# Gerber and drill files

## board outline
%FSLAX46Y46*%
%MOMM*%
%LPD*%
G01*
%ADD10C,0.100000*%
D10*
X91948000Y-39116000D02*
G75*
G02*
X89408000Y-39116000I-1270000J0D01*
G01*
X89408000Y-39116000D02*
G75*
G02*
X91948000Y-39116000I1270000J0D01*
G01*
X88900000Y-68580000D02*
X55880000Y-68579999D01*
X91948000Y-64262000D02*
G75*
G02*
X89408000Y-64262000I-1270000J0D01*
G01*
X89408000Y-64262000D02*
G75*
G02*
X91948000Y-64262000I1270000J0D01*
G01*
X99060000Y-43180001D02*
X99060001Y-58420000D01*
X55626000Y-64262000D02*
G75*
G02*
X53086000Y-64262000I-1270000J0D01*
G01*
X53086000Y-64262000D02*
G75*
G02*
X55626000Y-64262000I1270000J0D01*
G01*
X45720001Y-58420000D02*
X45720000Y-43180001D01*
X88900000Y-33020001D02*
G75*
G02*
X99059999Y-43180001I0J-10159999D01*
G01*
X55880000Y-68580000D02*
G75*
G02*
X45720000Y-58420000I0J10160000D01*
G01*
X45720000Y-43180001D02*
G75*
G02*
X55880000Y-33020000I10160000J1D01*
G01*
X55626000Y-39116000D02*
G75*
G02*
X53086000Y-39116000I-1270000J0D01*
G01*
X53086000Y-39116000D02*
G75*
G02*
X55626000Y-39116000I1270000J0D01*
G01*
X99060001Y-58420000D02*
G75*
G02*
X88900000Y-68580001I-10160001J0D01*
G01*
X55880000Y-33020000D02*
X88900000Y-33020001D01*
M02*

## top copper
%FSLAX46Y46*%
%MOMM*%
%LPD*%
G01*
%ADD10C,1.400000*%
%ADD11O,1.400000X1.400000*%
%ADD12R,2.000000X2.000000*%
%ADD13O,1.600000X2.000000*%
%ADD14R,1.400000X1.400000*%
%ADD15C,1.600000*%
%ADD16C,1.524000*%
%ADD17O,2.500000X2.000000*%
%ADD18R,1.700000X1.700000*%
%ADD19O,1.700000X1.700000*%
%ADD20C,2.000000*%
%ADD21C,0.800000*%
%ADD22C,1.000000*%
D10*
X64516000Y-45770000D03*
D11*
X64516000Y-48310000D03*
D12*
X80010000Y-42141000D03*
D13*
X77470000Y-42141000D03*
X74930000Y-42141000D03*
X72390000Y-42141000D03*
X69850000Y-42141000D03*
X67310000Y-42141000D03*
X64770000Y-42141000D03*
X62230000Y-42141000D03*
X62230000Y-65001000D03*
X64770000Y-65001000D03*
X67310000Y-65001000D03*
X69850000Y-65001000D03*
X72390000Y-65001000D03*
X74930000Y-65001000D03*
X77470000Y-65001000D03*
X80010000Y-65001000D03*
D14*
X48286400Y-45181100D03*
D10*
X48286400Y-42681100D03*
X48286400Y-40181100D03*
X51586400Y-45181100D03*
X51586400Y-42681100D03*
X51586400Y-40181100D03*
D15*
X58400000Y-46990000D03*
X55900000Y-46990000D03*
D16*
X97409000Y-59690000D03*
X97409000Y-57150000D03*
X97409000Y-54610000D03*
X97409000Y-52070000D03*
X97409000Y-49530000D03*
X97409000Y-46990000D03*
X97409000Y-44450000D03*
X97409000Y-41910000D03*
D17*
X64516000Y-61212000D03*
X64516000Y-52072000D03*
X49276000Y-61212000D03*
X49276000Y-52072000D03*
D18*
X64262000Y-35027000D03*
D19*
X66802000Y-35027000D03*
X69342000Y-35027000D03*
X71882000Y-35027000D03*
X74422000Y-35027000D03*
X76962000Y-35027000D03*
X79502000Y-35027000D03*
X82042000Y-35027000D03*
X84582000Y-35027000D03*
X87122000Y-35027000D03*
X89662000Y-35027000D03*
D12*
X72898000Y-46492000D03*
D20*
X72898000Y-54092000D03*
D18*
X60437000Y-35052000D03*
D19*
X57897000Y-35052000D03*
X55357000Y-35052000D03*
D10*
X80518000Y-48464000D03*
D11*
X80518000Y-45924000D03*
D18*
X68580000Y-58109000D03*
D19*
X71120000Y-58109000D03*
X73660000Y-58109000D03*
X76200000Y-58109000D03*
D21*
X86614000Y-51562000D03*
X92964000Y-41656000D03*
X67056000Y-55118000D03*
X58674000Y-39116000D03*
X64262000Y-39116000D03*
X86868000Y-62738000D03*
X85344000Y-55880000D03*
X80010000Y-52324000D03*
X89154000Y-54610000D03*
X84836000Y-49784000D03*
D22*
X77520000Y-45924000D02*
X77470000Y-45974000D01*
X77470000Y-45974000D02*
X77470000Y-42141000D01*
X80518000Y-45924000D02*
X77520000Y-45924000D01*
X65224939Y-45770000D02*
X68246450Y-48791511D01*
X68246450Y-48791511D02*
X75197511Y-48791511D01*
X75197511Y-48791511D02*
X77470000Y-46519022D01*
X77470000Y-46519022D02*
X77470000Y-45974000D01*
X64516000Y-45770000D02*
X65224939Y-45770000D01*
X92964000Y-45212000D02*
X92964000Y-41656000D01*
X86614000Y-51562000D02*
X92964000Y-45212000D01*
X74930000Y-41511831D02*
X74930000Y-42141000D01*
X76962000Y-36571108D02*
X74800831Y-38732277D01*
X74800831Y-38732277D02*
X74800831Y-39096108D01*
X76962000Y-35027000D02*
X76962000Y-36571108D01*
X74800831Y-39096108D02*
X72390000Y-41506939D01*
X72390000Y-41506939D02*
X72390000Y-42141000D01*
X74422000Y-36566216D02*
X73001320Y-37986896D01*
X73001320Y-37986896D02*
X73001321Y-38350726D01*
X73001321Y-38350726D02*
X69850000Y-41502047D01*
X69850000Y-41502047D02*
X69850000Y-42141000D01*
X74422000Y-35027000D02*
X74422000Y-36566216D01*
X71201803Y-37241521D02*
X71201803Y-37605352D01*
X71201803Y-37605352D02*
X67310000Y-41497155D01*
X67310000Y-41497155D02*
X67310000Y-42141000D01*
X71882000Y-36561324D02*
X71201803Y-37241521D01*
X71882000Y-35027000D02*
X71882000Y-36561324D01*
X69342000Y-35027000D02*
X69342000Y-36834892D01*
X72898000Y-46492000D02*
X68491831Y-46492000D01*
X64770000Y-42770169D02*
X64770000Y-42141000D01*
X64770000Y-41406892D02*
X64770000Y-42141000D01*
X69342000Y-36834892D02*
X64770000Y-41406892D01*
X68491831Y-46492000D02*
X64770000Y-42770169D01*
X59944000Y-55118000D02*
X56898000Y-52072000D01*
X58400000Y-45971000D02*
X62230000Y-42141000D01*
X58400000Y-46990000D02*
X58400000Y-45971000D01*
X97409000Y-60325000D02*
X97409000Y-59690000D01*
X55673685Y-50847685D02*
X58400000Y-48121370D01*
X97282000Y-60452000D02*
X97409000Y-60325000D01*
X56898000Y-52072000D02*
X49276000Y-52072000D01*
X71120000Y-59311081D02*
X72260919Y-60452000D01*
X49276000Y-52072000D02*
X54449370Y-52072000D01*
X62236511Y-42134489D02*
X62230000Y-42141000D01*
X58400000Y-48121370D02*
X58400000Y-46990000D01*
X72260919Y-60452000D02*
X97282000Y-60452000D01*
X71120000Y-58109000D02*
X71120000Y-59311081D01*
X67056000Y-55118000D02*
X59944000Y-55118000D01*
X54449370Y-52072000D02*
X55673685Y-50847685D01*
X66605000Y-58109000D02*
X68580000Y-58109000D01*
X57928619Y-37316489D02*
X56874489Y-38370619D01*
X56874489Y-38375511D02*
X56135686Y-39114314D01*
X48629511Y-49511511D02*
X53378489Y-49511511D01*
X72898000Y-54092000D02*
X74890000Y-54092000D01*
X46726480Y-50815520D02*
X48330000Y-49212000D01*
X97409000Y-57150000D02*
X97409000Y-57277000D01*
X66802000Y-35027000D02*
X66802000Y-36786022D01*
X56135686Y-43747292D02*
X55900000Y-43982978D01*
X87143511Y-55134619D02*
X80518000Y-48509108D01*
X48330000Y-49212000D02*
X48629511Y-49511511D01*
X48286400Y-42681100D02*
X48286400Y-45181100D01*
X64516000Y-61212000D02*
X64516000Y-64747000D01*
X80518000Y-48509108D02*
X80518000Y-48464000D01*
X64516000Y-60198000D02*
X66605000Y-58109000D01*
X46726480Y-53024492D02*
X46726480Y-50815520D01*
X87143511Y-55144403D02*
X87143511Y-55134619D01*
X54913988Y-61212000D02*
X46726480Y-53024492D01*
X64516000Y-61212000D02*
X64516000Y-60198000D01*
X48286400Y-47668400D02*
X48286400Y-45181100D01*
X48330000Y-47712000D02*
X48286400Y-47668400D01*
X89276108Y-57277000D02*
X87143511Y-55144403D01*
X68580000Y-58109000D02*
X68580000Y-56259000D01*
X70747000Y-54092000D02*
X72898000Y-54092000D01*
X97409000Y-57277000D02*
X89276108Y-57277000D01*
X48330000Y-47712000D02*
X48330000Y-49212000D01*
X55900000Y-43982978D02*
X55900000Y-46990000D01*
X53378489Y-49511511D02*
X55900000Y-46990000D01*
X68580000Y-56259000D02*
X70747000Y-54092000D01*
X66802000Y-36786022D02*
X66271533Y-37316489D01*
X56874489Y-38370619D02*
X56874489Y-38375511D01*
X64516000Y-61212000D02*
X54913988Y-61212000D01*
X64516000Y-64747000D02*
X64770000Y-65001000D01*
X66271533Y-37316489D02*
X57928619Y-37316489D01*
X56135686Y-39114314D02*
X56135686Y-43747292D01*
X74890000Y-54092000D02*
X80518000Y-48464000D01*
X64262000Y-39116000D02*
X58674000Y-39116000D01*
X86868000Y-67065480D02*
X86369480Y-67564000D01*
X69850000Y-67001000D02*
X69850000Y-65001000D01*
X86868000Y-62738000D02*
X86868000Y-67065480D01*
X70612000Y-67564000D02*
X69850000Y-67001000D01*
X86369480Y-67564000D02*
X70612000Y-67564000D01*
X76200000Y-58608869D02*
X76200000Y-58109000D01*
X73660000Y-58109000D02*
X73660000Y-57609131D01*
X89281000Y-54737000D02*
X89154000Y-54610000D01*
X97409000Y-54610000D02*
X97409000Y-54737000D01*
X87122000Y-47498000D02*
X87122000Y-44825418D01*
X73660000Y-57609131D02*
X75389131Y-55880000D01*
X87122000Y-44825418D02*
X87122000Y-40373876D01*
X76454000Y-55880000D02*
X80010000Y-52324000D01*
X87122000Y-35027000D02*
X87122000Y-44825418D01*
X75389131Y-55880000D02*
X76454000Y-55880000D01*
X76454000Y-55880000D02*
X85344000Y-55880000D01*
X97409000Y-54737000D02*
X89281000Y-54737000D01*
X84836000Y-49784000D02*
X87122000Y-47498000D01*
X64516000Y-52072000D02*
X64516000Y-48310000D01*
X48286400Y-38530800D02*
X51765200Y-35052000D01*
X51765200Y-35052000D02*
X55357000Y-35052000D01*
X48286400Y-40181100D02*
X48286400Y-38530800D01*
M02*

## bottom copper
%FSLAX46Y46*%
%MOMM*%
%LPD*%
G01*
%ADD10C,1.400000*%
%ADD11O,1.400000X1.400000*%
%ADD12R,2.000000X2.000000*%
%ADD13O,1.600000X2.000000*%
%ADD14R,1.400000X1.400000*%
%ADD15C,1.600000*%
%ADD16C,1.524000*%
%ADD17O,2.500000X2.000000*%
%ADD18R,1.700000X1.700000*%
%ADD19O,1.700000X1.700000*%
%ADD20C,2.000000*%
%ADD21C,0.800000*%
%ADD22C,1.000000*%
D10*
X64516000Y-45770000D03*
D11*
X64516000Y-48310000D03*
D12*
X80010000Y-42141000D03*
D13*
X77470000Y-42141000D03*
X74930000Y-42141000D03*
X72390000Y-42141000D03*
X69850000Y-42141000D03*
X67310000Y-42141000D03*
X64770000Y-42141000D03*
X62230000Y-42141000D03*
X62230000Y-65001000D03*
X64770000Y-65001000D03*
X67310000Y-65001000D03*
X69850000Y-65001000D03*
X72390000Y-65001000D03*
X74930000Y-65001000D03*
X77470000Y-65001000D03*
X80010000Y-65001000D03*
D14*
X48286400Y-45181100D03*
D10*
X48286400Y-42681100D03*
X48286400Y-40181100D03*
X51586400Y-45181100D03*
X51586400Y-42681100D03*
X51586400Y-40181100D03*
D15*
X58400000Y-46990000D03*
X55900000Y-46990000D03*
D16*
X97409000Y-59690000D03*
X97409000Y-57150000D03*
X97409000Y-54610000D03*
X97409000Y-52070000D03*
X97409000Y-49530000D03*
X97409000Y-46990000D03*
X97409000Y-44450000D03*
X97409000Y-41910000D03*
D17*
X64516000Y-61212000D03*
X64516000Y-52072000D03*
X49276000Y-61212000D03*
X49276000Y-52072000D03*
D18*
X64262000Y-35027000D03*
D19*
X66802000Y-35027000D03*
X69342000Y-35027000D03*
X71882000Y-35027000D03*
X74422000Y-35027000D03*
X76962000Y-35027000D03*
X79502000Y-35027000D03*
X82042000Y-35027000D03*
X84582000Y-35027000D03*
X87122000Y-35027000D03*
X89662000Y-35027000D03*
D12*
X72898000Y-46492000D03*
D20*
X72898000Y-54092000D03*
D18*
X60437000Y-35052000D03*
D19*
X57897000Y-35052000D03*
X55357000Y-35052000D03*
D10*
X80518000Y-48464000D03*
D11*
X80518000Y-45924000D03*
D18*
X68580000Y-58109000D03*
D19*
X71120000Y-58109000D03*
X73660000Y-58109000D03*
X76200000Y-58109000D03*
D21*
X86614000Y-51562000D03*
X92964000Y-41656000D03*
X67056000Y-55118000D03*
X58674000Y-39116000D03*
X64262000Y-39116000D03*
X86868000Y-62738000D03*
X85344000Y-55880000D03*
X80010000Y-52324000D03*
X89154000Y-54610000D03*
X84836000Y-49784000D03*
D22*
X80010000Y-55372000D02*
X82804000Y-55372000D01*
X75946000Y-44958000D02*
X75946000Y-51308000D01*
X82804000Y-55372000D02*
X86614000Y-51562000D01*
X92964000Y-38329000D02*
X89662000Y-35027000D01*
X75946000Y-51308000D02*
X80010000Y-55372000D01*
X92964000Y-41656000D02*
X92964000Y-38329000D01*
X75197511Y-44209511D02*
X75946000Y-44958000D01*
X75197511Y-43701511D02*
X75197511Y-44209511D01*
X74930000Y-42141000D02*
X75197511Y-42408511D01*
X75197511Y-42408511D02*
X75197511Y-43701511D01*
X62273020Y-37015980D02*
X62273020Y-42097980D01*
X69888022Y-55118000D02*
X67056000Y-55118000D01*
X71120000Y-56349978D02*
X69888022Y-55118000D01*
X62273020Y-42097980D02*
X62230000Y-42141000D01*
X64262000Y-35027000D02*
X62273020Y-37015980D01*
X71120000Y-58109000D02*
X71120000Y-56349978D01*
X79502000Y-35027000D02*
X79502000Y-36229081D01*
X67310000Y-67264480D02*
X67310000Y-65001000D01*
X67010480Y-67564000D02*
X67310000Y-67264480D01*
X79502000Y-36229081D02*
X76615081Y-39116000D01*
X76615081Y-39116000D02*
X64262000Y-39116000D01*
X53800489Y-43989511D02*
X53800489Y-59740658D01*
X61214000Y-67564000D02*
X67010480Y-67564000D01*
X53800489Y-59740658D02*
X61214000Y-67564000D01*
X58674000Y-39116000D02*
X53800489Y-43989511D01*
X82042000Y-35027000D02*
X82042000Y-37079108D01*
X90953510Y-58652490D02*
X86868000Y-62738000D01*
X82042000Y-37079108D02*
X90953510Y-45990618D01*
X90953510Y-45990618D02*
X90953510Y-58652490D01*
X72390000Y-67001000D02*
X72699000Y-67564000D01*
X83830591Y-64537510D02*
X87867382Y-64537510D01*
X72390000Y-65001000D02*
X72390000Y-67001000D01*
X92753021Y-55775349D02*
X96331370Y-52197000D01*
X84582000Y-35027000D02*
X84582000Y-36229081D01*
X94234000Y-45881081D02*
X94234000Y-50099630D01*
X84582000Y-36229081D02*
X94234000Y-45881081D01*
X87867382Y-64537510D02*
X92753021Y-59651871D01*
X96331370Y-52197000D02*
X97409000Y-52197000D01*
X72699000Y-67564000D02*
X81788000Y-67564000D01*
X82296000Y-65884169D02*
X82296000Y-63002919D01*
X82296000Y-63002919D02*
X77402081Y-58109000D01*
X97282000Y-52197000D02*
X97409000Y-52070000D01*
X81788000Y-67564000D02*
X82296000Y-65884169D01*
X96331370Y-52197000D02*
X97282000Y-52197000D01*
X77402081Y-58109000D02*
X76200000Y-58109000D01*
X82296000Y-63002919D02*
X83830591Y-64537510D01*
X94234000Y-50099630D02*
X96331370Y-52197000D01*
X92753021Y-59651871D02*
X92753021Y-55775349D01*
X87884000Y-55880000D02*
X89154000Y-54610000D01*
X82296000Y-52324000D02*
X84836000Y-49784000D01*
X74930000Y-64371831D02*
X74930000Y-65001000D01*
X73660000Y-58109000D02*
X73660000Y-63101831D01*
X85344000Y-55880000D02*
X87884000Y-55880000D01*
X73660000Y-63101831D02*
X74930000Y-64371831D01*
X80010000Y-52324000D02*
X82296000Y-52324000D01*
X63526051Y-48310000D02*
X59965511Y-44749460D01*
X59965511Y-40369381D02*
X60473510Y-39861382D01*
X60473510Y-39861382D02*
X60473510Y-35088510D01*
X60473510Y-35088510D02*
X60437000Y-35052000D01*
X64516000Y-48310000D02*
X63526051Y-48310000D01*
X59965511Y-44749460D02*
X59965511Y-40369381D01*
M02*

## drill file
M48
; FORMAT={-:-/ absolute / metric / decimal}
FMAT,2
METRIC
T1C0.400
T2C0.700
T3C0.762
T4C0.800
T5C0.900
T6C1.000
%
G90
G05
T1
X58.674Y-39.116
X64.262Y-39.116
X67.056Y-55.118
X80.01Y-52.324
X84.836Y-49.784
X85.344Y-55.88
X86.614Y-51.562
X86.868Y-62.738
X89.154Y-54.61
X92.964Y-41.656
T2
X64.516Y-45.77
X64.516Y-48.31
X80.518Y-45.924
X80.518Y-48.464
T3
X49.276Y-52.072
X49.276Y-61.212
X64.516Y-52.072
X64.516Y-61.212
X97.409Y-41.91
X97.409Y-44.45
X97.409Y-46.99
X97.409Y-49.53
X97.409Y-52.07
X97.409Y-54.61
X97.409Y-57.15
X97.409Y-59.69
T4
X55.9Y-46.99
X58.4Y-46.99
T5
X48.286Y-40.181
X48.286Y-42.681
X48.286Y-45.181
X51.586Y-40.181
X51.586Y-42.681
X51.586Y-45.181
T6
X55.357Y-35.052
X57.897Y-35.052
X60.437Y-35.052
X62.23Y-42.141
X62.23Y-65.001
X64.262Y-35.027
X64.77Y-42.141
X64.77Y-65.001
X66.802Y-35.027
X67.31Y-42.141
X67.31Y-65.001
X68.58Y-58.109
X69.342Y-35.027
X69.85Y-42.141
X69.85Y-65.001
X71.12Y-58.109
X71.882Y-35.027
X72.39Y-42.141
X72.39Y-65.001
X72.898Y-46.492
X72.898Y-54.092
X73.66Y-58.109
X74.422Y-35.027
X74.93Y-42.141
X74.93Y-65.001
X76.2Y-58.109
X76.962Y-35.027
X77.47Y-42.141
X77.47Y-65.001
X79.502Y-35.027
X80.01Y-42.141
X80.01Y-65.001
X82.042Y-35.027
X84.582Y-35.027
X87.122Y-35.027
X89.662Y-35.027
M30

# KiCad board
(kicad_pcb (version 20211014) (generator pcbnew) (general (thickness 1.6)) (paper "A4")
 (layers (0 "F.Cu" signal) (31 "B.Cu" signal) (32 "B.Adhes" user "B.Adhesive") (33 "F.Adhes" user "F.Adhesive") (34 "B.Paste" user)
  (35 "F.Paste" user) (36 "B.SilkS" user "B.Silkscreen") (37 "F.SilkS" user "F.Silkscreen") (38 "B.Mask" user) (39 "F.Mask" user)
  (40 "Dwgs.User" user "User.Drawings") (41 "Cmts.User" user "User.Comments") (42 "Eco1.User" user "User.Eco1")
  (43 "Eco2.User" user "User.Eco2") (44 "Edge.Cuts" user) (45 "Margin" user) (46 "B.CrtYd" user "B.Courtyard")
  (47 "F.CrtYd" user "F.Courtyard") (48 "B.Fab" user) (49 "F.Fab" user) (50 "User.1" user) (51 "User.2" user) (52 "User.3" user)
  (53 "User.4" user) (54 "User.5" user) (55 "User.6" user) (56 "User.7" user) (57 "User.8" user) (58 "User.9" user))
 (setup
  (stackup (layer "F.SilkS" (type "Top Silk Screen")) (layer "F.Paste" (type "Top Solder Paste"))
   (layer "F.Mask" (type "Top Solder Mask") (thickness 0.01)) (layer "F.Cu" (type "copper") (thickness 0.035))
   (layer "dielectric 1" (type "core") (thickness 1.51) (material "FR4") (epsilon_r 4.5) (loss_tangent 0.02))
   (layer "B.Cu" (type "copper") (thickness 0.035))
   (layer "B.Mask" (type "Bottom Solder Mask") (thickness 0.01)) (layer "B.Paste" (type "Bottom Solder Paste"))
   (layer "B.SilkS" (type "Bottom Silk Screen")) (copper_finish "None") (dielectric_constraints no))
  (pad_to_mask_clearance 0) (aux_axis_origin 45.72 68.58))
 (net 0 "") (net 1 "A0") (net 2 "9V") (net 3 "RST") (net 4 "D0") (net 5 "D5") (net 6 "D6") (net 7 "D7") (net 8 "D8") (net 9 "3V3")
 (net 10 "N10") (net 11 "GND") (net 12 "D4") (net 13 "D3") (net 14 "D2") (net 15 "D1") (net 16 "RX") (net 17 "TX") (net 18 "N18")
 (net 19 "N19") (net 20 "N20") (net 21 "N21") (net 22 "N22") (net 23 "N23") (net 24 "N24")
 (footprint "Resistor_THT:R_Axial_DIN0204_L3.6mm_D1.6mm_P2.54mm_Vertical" (layer "F.Cu") (at 64.516 45.77 -90)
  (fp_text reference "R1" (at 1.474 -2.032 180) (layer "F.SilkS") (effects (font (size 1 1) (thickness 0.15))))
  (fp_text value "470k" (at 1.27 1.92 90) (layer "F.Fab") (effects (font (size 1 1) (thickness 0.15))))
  (pad "1" thru_hole circle (at 0 0 270) (size 1.4 1.4) (drill 0.7) (layers *.Cu *.Mask) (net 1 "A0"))
  (pad "2" thru_hole oval (at 2.54 0 270) (size 1.4 1.4) (drill 0.7) (layers *.Cu *.Mask) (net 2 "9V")))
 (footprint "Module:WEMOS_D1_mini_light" (layer "F.Cu") (at 80.01 42.141 -90)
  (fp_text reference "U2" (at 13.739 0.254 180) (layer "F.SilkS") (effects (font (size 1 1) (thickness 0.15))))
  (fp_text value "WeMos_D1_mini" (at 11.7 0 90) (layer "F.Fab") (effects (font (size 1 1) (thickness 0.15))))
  (pad "1" thru_hole rect (at 0 0 270) (size 2 2) (drill 1) (layers *.Cu *.Mask) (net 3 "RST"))
  (pad "2" thru_hole oval (at 0 2.54 270) (size 2 1.6) (drill 1) (layers *.Cu *.Mask) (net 1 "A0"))
  (pad "3" thru_hole oval (at 0 5.08 270) (size 2 1.6) (drill 1) (layers *.Cu *.Mask) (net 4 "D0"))
  (pad "4" thru_hole oval (at 0 7.62 270) (size 2 1.6) (drill 1) (layers *.Cu *.Mask) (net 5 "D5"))
  (pad "5" thru_hole oval (at 0 10.16 270) (size 2 1.6) (drill 1) (layers *.Cu *.Mask) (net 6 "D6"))
  (pad "6" thru_hole oval (at 0 12.7 270) (size 2 1.6) (drill 1) (layers *.Cu *.Mask) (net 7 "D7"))
  (pad "7" thru_hole oval (at 0 15.24 270) (size 2 1.6) (drill 1) (layers *.Cu *.Mask) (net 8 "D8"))
  (pad "8" thru_hole oval (at 0 17.78 270) (size 2 1.6) (drill 1) (layers *.Cu *.Mask) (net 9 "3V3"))
  (pad "9" thru_hole oval (at 22.86 17.78 270) (size 2 1.6) (drill 1) (layers *.Cu *.Mask) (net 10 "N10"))
  (pad "10" thru_hole oval (at 22.86 15.24 270) (size 2 1.6) (drill 1) (layers *.Cu *.Mask) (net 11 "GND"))
  (pad "11" thru_hole oval (at 22.86 12.7 270) (size 2 1.6) (drill 1) (layers *.Cu *.Mask) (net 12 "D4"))
  (pad "12" thru_hole oval (at 22.86 10.16 270) (size 2 1.6) (drill 1) (layers *.Cu *.Mask) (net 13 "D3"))
  (pad "13" thru_hole oval (at 22.86 7.62 270) (size 2 1.6) (drill 1) (layers *.Cu *.Mask) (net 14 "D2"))
  (pad "14" thru_hole oval (at 22.86 5.08 270) (size 2 1.6) (drill 1) (layers *.Cu *.Mask) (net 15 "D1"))
  (pad "15" thru_hole oval (at 22.86 2.54 270) (size 2 1.6) (drill 1) (layers *.Cu *.Mask) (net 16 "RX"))
  (pad "16" thru_hole oval (at 22.86 0 270) (size 2 1.6) (drill 1) (layers *.Cu *.Mask) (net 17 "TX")))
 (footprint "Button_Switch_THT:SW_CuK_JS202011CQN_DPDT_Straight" (layer "F.Cu") (at 48.2864 45.1811 90)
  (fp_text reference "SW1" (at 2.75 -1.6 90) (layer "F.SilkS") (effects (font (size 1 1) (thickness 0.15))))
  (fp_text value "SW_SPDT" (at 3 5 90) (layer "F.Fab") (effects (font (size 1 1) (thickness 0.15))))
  (pad "1" thru_hole rect (at 0 0 90) (size 1.4 1.4) (drill 0.9) (layers *.Cu *.Mask) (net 11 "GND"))
  (pad "2" thru_hole circle (at 2.5 0 90) (size 1.4 1.4) (drill 0.9) (layers *.Cu *.Mask) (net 11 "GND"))
  (pad "3" thru_hole circle (at 5 0 90) (size 1.4 1.4) (drill 0.9) (layers *.Cu *.Mask) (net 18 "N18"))
  (pad "4" thru_hole circle (at 0 3.3 90) (size 1.4 1.4) (drill 0.9) (layers *.Cu *.Mask))
  (pad "5" thru_hole circle (at 2.5 3.3 90) (size 1.4 1.4) (drill 0.9) (layers *.Cu *.Mask))
  (pad "6" thru_hole circle (at 5 3.3 90) (size 1.4 1.4) (drill 0.9) (layers *.Cu *.Mask)))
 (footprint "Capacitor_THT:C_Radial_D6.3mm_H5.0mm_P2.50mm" (layer "F.Cu") (at 58.4 46.99 180)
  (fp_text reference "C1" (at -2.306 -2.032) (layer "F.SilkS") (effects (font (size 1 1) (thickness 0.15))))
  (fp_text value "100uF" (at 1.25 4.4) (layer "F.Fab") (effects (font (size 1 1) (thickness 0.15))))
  (pad "1" thru_hole circle (at 0 0 180) (size 1.6 1.6) (drill 0.8) (layers *.Cu *.Mask) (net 9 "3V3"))
  (pad "2" thru_hole circle (at 2.5 0 180) (size 1.6 1.6) (drill 0.8) (layers *.Cu *.Mask) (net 11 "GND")))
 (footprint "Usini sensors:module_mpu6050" (layer "F.Cu") (at 97.409 41.91 180)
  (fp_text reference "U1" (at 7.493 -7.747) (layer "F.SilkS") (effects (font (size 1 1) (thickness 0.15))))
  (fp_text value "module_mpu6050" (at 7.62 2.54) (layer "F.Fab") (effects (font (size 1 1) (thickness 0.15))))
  (pad "1" thru_hole circle locked (at 0 -17.78 180) (size 1.524 1.524) (drill 0.762) (layers *.Cu *.Mask) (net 9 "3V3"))
  (pad "2" thru_hole circle locked (at 0 -15.24 180) (size 1.524 1.524) (drill 0.762) (layers *.Cu *.Mask) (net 11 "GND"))
  (pad "3" thru_hole circle locked (at 0 -12.7 180) (size 1.524 1.524) (drill 0.762) (layers *.Cu *.Mask) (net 15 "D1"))
  (pad "4" thru_hole circle locked (at 0 -10.16 180) (size 1.524 1.524) (drill 0.762) (layers *.Cu *.Mask) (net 14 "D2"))
  (pad "5" thru_hole circle locked (at 0 -7.62 180) (size 1.524 1.524) (drill 0.762) (layers *.Cu *.Mask) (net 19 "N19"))
  (pad "6" thru_hole circle locked (at 0 -5.08 180) (size 1.524 1.524) (drill 0.762) (layers *.Cu *.Mask) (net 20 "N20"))
  (pad "7" thru_hole circle locked (at 0 -2.54 180) (size 1.524 1.524) (drill 0.762) (layers *.Cu *.Mask) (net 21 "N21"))
  (pad "8" thru_hole circle locked (at 0 0 180) (size 1.524 1.524) (drill 0.762) (layers *.Cu *.Mask) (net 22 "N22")))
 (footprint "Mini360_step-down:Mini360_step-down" (layer "F.Cu") (at 56.896 56.642 180)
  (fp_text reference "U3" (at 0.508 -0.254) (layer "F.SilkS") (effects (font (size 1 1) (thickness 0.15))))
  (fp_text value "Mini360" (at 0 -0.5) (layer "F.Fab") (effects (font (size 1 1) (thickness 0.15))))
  (pad "1" thru_hole oval locked (at -7.62 -4.57 180) (size 2.5 2) (drill 0.762) (layers *.Cu *.Mask) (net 11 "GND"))
  (pad "2" thru_hole oval locked (at -7.62 4.57 180) (size 2.5 2) (drill 0.762) (layers *.Cu *.Mask) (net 2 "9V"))
  (pad "3" thru_hole oval locked (at 7.62 -4.57 180) (size 2.5 2) (drill 0.762) (layers *.Cu *.Mask) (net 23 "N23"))
  (pad "4" thru_hole oval locked (at 7.62 4.57 180) (size 2.5 2) (drill 0.762) (layers *.Cu *.Mask) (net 9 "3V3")))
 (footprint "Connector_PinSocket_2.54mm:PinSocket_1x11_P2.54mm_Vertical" (layer "F.Cu") (at 64.262 35.027 90)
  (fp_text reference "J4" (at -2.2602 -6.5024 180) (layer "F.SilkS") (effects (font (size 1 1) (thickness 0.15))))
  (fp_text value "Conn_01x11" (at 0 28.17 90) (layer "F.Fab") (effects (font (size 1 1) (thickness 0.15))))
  (pad "1" thru_hole rect (at 0 0 90) (size 1.7 1.7) (drill 1) (layers *.Cu *.Mask) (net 9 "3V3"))
  (pad "2" thru_hole oval (at 0 2.54 90) (size 1.7 1.7) (drill 1) (layers *.Cu *.Mask) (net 11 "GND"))
  (pad "3" thru_hole oval (at 0 5.08 90) (size 1.7 1.7) (drill 1) (layers *.Cu *.Mask) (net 8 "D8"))
  (pad "4" thru_hole oval (at 0 7.62 90) (size 1.7 1.7) (drill 1) (layers *.Cu *.Mask) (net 7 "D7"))
  (pad "5" thru_hole oval (at 0 10.16 90) (size 1.7 1.7) (drill 1) (layers *.Cu *.Mask) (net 6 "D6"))
  (pad "6" thru_hole oval (at 0 12.7 90) (size 1.7 1.7) (drill 1) (layers *.Cu *.Mask) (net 5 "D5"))
  (pad "7" thru_hole oval (at 0 15.24 90) (size 1.7 1.7) (drill 1) (layers *.Cu *.Mask) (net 12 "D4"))
  (pad "8" thru_hole oval (at 0 17.78 90) (size 1.7 1.7) (drill 1) (layers *.Cu *.Mask) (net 13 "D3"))
  (pad "9" thru_hole oval (at 0 20.32 90) (size 1.7 1.7) (drill 1) (layers *.Cu *.Mask) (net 14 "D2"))
  (pad "10" thru_hole oval (at 0 22.86 90) (size 1.7 1.7) (drill 1) (layers *.Cu *.Mask) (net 15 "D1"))
  (pad "11" thru_hole oval (at 0 25.4 90) (size 1.7 1.7) (drill 1) (layers *.Cu *.Mask) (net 4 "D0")))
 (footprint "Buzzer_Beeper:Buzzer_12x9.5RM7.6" (layer "F.Cu") (at 72.898 46.492 -90)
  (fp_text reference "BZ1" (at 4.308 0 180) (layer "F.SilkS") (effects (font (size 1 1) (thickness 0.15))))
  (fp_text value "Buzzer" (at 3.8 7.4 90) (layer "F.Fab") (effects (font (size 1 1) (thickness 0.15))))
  (pad "1" thru_hole rect (at 0 0 270) (size 2 2) (drill 1) (layers *.Cu *.Mask) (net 8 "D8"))
  (pad "2" thru_hole circle (at 7.6 0 270) (size 2 2) (drill 1) (layers *.Cu *.Mask) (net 11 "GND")))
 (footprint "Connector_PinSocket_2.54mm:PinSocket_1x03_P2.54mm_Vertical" (layer "F.Cu") (at 60.437 35.052 -90)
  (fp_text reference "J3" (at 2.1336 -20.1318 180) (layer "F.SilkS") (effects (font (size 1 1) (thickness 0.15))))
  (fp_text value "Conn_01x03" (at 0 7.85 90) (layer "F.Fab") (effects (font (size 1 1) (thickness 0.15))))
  (pad "1" thru_hole rect (at 0 0 270) (size 1.7 1.7) (drill 1) (layers *.Cu *.Mask) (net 2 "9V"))
  (pad "2" thru_hole oval (at 0 2.54 270) (size 1.7 1.7) (drill 1) (layers *.Cu *.Mask) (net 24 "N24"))
  (pad "3" thru_hole oval (at 0 5.08 270) (size 1.7 1.7) (drill 1) (layers *.Cu *.Mask) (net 18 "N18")))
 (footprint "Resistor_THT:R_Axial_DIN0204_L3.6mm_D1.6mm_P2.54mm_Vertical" (layer "F.Cu") (at 80.518 48.464 90)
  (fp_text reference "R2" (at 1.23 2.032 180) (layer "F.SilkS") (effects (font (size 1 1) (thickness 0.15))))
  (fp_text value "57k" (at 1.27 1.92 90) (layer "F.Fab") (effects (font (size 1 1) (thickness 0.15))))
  (pad "1" thru_hole circle (at 0 0 90) (size 1.4 1.4) (drill 0.7) (layers *.Cu *.Mask) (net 11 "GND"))
  (pad "2" thru_hole oval (at 2.54 0 90) (size 1.4 1.4) (drill 0.7) (layers *.Cu *.Mask) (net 1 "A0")))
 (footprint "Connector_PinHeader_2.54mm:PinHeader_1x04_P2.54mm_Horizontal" (layer "B.Cu") (at 68.58 58.109 -90)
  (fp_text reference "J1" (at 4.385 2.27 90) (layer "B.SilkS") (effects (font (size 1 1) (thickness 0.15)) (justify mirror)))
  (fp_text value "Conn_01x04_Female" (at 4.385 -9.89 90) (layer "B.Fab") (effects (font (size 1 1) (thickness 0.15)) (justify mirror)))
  (pad "1" thru_hole rect (at 0 0 270) (size 1.7 1.7) (drill 1) (layers *.Cu *.Mask) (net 11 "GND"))
  (pad "2" thru_hole oval (at 0 -2.54 270) (size 1.7 1.7) (drill 1) (layers *.Cu *.Mask) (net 9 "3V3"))
  (pad "3" thru_hole oval (at 0 -5.08 270) (size 1.7 1.7) (drill 1) (layers *.Cu *.Mask) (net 15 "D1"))
  (pad "4" thru_hole oval (at 0 -7.62 270) (size 1.7 1.7) (drill 1) (layers *.Cu *.Mask) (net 14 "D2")))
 (gr_circle (center 90.678 39.116) (end 91.948 39.116) (layer "Edge.Cuts") (width 0.1) (fill none))
 (gr_line (start 88.9 68.58) (end 55.88 68.579999) (layer "Edge.Cuts") (width 0.1))
 (gr_circle (center 90.678 64.262) (end 91.948 64.262) (layer "Edge.Cuts") (width 0.1) (fill none))
 (gr_line (start 99.06 43.180001) (end 99.060001 58.42) (layer "Edge.Cuts") (width 0.1))
 (gr_circle (center 54.356 64.262) (end 55.626 64.262) (layer "Edge.Cuts") (width 0.1) (fill none))
 (gr_line (start 45.720001 58.42) (end 45.72 43.180001) (layer "Edge.Cuts") (width 0.1))
 (gr_arc (start 88.9 33.020001) (mid 96.084205 35.995796) (end 99.06 43.180001) (layer "Edge.Cuts") (width 0.1))
 (gr_arc (start 55.88 68.58) (mid 48.695795 65.604205) (end 45.72 58.42) (layer "Edge.Cuts") (width 0.1))
 (gr_arc (start 45.72 43.180001) (mid 48.695795 35.995796) (end 55.88 33.020001) (layer "Edge.Cuts") (width 0.1))
 (gr_circle (center 54.356 39.116) (end 55.626 39.116) (layer "Edge.Cuts") (width 0.1) (fill none))
 (gr_arc (start 99.060001 58.42) (mid 96.084206 65.604206) (end 88.9 68.580001) (layer "Edge.Cuts") (width 0.1))
 (gr_line (start 55.88 33.02) (end 88.9 33.020001) (layer "Edge.Cuts") (width 0.1))
 (segment (start 77.52 45.924) (end 77.47 45.974) (width 1) (layer "F.Cu") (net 1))
 (segment (start 77.47 45.974) (end 77.47 42.141) (width 1) (layer "F.Cu") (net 1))
 (segment (start 80.518 45.924) (end 77.52 45.924) (width 1) (layer "F.Cu") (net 1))
 (segment (start 65.224939 45.77) (end 68.24645 48.791511) (width 1) (layer "F.Cu") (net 1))
 (segment (start 68.24645 48.791511) (end 75.197511 48.791511) (width 1) (layer "F.Cu") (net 1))
 (segment (start 75.197511 48.791511) (end 77.47 46.519022) (width 1) (layer "F.Cu") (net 1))
 (segment (start 77.47 46.519022) (end 77.47 45.974) (width 1) (layer "F.Cu") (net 1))
 (segment (start 64.516 45.77) (end 65.224939 45.77) (width 1) (layer "F.Cu") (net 1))
 (segment (start 92.964 45.212) (end 92.964 41.656) (width 1) (layer "F.Cu") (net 4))
 (segment (start 86.614 51.562) (end 92.964 45.212) (width 1) (layer "F.Cu") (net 4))
 (segment (start 74.93 41.511831) (end 74.93 42.141) (width 1) (layer "F.Cu") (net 4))
 (via (at 86.614 51.562) (size 0.8) (drill 0.4) (layers "F.Cu" "B.Cu") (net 4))
 (via (at 92.964 41.656) (size 0.8) (drill 0.4) (layers "F.Cu" "B.Cu") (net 4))
 (segment (start 80.01 55.372) (end 82.804 55.372) (width 1) (layer "B.Cu") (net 4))
 (segment (start 75.946 44.958) (end 75.946 51.308) (width 1) (layer "B.Cu") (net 4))
 (segment (start 82.804 55.372) (end 86.614 51.562) (width 1) (layer "B.Cu") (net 4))
 (segment (start 92.964 38.329) (end 89.662 35.027) (width 1) (layer "B.Cu") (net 4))
 (segment (start 75.946 51.308) (end 80.01 55.372) (width 1) (layer "B.Cu") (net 4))
 (segment (start 92.964 41.656) (end 92.964 38.329) (width 1) (layer "B.Cu") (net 4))
 (segment (start 75.197511 44.209511) (end 75.946 44.958) (width 1) (layer "B.Cu") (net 4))
 (segment (start 75.197511 43.701511) (end 75.197511 44.209511) (width 1) (layer "B.Cu") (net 4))
 (segment (start 74.93 42.141) (end 75.197511 42.408511) (width 1) (layer "B.Cu") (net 4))
 (segment (start 75.197511 42.408511) (end 75.197511 43.701511) (width 1) (layer "B.Cu") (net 4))
 (segment (start 76.962 36.571108) (end 74.800831 38.732277) (width 1) (layer "F.Cu") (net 5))
 (segment (start 74.800831 38.732277) (end 74.800831 39.096108) (width 1) (layer "F.Cu") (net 5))
 (segment (start 76.962 35.027) (end 76.962 36.571108) (width 1) (layer "F.Cu") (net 5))
 (segment (start 74.800831 39.096108) (end 72.39 41.506939) (width 1) (layer "F.Cu") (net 5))
 (segment (start 72.39 41.506939) (end 72.39 42.141) (width 1) (layer "F.Cu") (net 5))
 (segment (start 74.422 36.566216) (end 73.00132 37.986896) (width 1) (layer "F.Cu") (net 6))
 (segment (start 73.00132 37.986896) (end 73.001321 38.350726) (width 1) (layer "F.Cu") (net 6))
 (segment (start 73.001321 38.350726) (end 69.85 41.502047) (width 1) (layer "F.Cu") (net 6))
 (segment (start 69.85 41.502047) (end 69.85 42.141) (width 1) (layer "F.Cu") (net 6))
 (segment (start 74.422 35.027) (end 74.422 36.566216) (width 1) (layer "F.Cu") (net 6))
 (segment (start 71.201803 37.241521) (end 71.201803 37.605352) (width 1) (layer "F.Cu") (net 7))
 (segment (start 71.201803 37.605352) (end 67.31 41.497155) (width 1) (layer "F.Cu") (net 7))
 (segment (start 67.31 41.497155) (end 67.31 42.141) (width 1) (layer "F.Cu") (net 7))
 (segment (start 71.882 36.561324) (end 71.201803 37.241521) (width 1) (layer "F.Cu") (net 7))
 (segment (start 71.882 35.027) (end 71.882 36.561324) (width 1) (layer "F.Cu") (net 7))
 (segment (start 69.342 35.027) (end 69.342 36.834892) (width 1) (layer "F.Cu") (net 8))
 (segment (start 72.898 46.492) (end 68.491831 46.492) (width 1) (layer "F.Cu") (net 8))
 (segment (start 64.77 42.770169) (end 64.77 42.141) (width 1) (layer "F.Cu") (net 8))
 (segment (start 64.77 41.406892) (end 64.77 42.141) (width 1) (layer "F.Cu") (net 8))
 (segment (start 69.342 36.834892) (end 64.77 41.406892) (width 1) (layer "F.Cu") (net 8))
 (segment (start 68.491831 46.492) (end 64.77 42.770169) (width 1) (layer "F.Cu") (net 8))
 (segment (start 59.944 55.118) (end 56.898 52.072) (width 1) (layer "F.Cu") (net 9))
 (segment (start 58.4 45.971) (end 62.23 42.141) (width 1) (layer "F.Cu") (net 9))
 (segment (start 58.4 46.99) (end 58.4 45.971) (width 1) (layer "F.Cu") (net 9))
 (segment (start 97.409 60.325) (end 97.409 59.69) (width 1) (layer "F.Cu") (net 9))
 (segment (start 55.673685 50.847685) (end 58.4 48.12137) (width 1) (layer "F.Cu") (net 9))
 (segment (start 97.282 60.452) (end 97.409 60.325) (width 1) (layer "F.Cu") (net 9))
 (segment (start 56.898 52.072) (end 49.276 52.072) (width 1) (layer "F.Cu") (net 9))
 (segment (start 71.12 59.311081) (end 72.260919 60.452) (width 1) (layer "F.Cu") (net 9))
 (segment (start 49.276 52.072) (end 54.44937 52.072) (width 1) (layer "F.Cu") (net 9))
 (segment (start 62.236511 42.134489) (end 62.23 42.141) (width 1) (layer "F.Cu") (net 9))
 (segment (start 58.4 48.12137) (end 58.4 46.99) (width 1) (layer "F.Cu") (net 9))
 (segment (start 72.260919 60.452) (end 97.282 60.452) (width 1) (layer "F.Cu") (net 9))
 (segment (start 71.12 58.109) (end 71.12 59.311081) (width 1) (layer "F.Cu") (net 9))
 (segment (start 67.056 55.118) (end 59.944 55.118) (width 1) (layer "F.Cu") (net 9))
 (segment (start 54.44937 52.072) (end 55.673685 50.847685) (width 1) (layer "F.Cu") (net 9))
 (via (at 67.056 55.118) (size 0.8) (drill 0.4) (layers "F.Cu" "B.Cu") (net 9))
 (segment (start 62.27302 37.01598) (end 62.27302 42.09798) (width 1) (layer "B.Cu") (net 9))
 (segment (start 69.888022 55.118) (end 67.056 55.118) (width 1) (layer "B.Cu") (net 9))
 (segment (start 71.12 56.349978) (end 69.888022 55.118) (width 1) (layer "B.Cu") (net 9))
 (segment (start 62.27302 42.09798) (end 62.23 42.141) (width 1) (layer "B.Cu") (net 9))
 (segment (start 64.262 35.027) (end 62.27302 37.01598) (width 1) (layer "B.Cu") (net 9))
 (segment (start 71.12 58.109) (end 71.12 56.349978) (width 1) (layer "B.Cu") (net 9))
 (segment (start 66.605 58.109) (end 68.58 58.109) (width 1) (layer "F.Cu") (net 11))
 (segment (start 57.928619 37.316489) (end 56.874489 38.370619) (width 1) (layer "F.Cu") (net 11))
 (segment (start 56.874489 38.375511) (end 56.135686 39.114314) (width 1) (layer "F.Cu") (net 11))
 (segment (start 48.629511 49.511511) (end 53.378489 49.511511) (width 1) (layer "F.Cu") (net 11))
 (segment (start 72.898 54.092) (end 74.89 54.092) (width 1) (layer "F.Cu") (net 11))
 (segment (start 46.72648 50.81552) (end 48.33 49.212) (width 1) (layer "F.Cu") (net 11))
 (segment (start 97.409 57.15) (end 97.409 57.277) (width 1) (layer "F.Cu") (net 11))
 (segment (start 66.802 35.027) (end 66.802 36.786022) (width 1) (layer "F.Cu") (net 11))
 (segment (start 56.135686 43.747292) (end 55.9 43.982978) (width 1) (layer "F.Cu") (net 11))
 (segment (start 87.143511 55.134619) (end 80.518 48.509108) (width 1) (layer "F.Cu") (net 11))
 (segment (start 48.33 49.212) (end 48.629511 49.511511) (width 1) (layer "F.Cu") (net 11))
 (segment (start 48.2864 42.6811) (end 48.2864 45.1811) (width 1) (layer "F.Cu") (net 11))
 (segment (start 64.516 61.212) (end 64.516 64.747) (width 1) (layer "F.Cu") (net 11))
 (segment (start 80.518 48.509108) (end 80.518 48.464) (width 1) (layer "F.Cu") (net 11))
 (segment (start 64.516 60.198) (end 66.605 58.109) (width 1) (layer "F.Cu") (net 11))
 (segment (start 46.72648 53.024492) (end 46.72648 50.81552) (width 1) (layer "F.Cu") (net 11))
 (segment (start 87.143511 55.144403) (end 87.143511 55.134619) (width 1) (layer "F.Cu") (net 11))
 (segment (start 54.913988 61.212) (end 46.72648 53.024492) (width 1) (layer "F.Cu") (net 11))
 (segment (start 64.516 61.212) (end 64.516 60.198) (width 1) (layer "F.Cu") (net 11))
 (segment (start 48.2864 47.6684) (end 48.2864 45.1811) (width 1) (layer "F.Cu") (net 11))
 (segment (start 48.33 47.712) (end 48.2864 47.6684) (width 1) (layer "F.Cu") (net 11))
 (segment (start 89.276108 57.277) (end 87.143511 55.144403) (width 1) (layer "F.Cu") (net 11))
 (segment (start 68.58 58.109) (end 68.58 56.259) (width 1) (layer "F.Cu") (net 11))
 (segment (start 70.747 54.092) (end 72.898 54.092) (width 1) (layer "F.Cu") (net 11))
 (segment (start 97.409 57.277) (end 89.276108 57.277) (width 1) (layer "F.Cu") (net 11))
 (segment (start 48.33 47.712) (end 48.33 49.212) (width 1) (layer "F.Cu") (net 11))
 (segment (start 55.9 43.982978) (end 55.9 46.99) (width 1) (layer "F.Cu") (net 11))
 (segment (start 53.378489 49.511511) (end 55.9 46.99) (width 1) (layer "F.Cu") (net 11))
 (segment (start 68.58 56.259) (end 70.747 54.092) (width 1) (layer "F.Cu") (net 11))
 (segment (start 66.802 36.786022) (end 66.271533 37.316489) (width 1) (layer "F.Cu") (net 11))
 (segment (start 56.874489 38.370619) (end 56.874489 38.375511) (width 1) (layer "F.Cu") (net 11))
 (segment (start 64.516 61.212) (end 54.913988 61.212) (width 1) (layer "F.Cu") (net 11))
 (segment (start 64.516 64.747) (end 64.77 65.001) (width 1) (layer "F.Cu") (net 11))
 (segment (start 66.271533 37.316489) (end 57.928619 37.316489) (width 1) (layer "F.Cu") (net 11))
 (segment (start 56.135686 39.114314) (end 56.135686 43.747292) (width 1) (layer "F.Cu") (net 11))
 (segment (start 74.89 54.092) (end 80.518 48.464) (width 1) (layer "F.Cu") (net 11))
 (segment (start 64.262 39.116) (end 58.674 39.116) (width 1) (layer "F.Cu") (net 12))
 (via (at 58.674 39.116) (size 0.8) (drill 0.4) (layers "F.Cu" "B.Cu") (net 12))
 (via (at 64.262 39.116) (size 0.8) (drill 0.4) (layers "F.Cu" "B.Cu") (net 12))
 (segment (start 79.502 35.027) (end 79.502 36.229081) (width 1) (layer "B.Cu") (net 12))
 (segment (start 67.31 67.26448) (end 67.31 65.001) (width 1) (layer "B.Cu") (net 12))
 (segment (start 67.01048 67.564) (end 67.31 67.26448) (width 1) (layer "B.Cu") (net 12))
 (segment (start 79.502 36.229081) (end 76.615081 39.116) (width 1) (layer "B.Cu") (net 12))
 (segment (start 76.615081 39.116) (end 64.262 39.116) (width 1) (layer "B.Cu") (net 12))
 (segment (start 53.800489 43.989511) (end 53.800489 59.740658) (width 1) (layer "B.Cu") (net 12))
 (segment (start 61.214 67.564) (end 67.01048 67.564) (width 1) (layer "B.Cu") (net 12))
 (segment (start 53.800489 59.740658) (end 61.214 67.564) (width 1) (layer "B.Cu") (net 12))
 (segment (start 58.674 39.116) (end 53.800489 43.989511) (width 1) (layer "B.Cu") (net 12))
 (segment (start 86.868 67.06548) (end 86.36948 67.564) (width 1) (layer "F.Cu") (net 13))
 (segment (start 69.85 67.001) (end 69.85 65.001) (width 1) (layer "F.Cu") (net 13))
 (segment (start 86.868 62.738) (end 86.868 67.06548) (width 1) (layer "F.Cu") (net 13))
 (segment (start 70.612 67.564) (end 69.85 67.001) (width 1) (layer "F.Cu") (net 13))
 (segment (start 86.36948 67.564) (end 70.612 67.564) (width 1) (layer "F.Cu") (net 13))
 (via (at 86.868 62.738) (size 0.8) (drill 0.4) (layers "F.Cu" "B.Cu") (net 13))
 (segment (start 82.042 35.027) (end 82.042 37.079108) (width 1) (layer "B.Cu") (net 13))
 (segment (start 90.95351 58.65249) (end 86.868 62.738) (width 1) (layer "B.Cu") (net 13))
 (segment (start 82.042 37.079108) (end 90.95351 45.990618) (width 1) (layer "B.Cu") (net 13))
 (segment (start 90.95351 45.990618) (end 90.95351 58.65249) (width 1) (layer "B.Cu") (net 13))
 (segment (start 76.2 58.608869) (end 76.2 58.109) (width 1) (layer "F.Cu") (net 14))
 (segment (start 72.39 67.001) (end 72.699 67.564) (width 1) (layer "B.Cu") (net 14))
 (segment (start 83.830591 64.53751) (end 87.867382 64.53751) (width 1) (layer "B.Cu") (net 14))
 (segment (start 72.39 65.001) (end 72.39 67.001) (width 1) (layer "B.Cu") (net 14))
 (segment (start 92.753021 55.775349) (end 96.33137 52.197) (width 1) (layer "B.Cu") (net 14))
 (segment (start 84.582 35.027) (end 84.582 36.229081) (width 1) (layer "B.Cu") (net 14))
 (segment (start 94.234 45.881081) (end 94.234 50.09963) (width 1) (layer "B.Cu") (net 14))
 (segment (start 84.582 36.229081) (end 94.234 45.881081) (width 1) (layer "B.Cu") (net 14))
 (segment (start 87.867382 64.53751) (end 92.753021 59.651871) (width 1) (layer "B.Cu") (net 14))
 (segment (start 96.33137 52.197) (end 97.409 52.197) (width 1) (layer "B.Cu") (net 14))
 (segment (start 72.699 67.564) (end 81.788 67.564) (width 1) (layer "B.Cu") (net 14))
 (segment (start 82.296 65.884169) (end 82.296 63.002919) (width 1) (layer "B.Cu") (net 14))
 (segment (start 82.296 63.002919) (end 77.402081 58.109) (width 1) (layer "B.Cu") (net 14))
 (segment (start 97.282 52.197) (end 97.409 52.07) (width 1) (layer "B.Cu") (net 14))
 (segment (start 81.788 67.564) (end 82.296 65.884169) (width 1) (layer "B.Cu") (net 14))
 (segment (start 96.33137 52.197) (end 97.282 52.197) (width 1) (layer "B.Cu") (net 14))
 (segment (start 77.402081 58.109) (end 76.2 58.109) (width 1) (layer "B.Cu") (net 14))
 (segment (start 82.296 63.002919) (end 83.830591 64.53751) (width 1) (layer "B.Cu") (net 14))
 (segment (start 94.234 50.09963) (end 96.33137 52.197) (width 1) (layer "B.Cu") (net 14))
 (segment (start 92.753021 59.651871) (end 92.753021 55.775349) (width 1) (layer "B.Cu") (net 14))
 (segment (start 73.66 58.109) (end 73.66 57.609131) (width 1) (layer "F.Cu") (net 15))
 (segment (start 89.281 54.737) (end 89.154 54.61) (width 1) (layer "F.Cu") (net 15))
 (segment (start 97.409 54.61) (end 97.409 54.737) (width 1) (layer "F.Cu") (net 15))
 (segment (start 87.122 47.498) (end 87.122 44.825418) (width 1) (layer "F.Cu") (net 15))
 (segment (start 73.66 57.609131) (end 75.389131 55.88) (width 1) (layer "F.Cu") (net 15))
 (segment (start 87.122 44.825418) (end 87.122 40.373876) (width 1) (layer "F.Cu") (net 15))
 (segment (start 76.454 55.88) (end 80.01 52.324) (width 1) (layer "F.Cu") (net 15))
 (segment (start 87.122 35.027) (end 87.122 44.825418) (width 1) (layer "F.Cu") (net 15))
 (segment (start 75.389131 55.88) (end 76.454 55.88) (width 1) (layer "F.Cu") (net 15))
 (segment (start 76.454 55.88) (end 85.344 55.88) (width 1) (layer "F.Cu") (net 15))
 (segment (start 97.409 54.737) (end 89.281 54.737) (width 1) (layer "F.Cu") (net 15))
 (segment (start 84.836 49.784) (end 87.122 47.498) (width 1) (layer "F.Cu") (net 15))
 (via (at 85.344 55.88) (size 0.8) (drill 0.4) (layers "F.Cu" "B.Cu") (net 15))
 (via (at 80.01 52.324) (size 0.8) (drill 0.4) (layers "F.Cu" "B.Cu") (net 15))
 (via (at 89.154 54.61) (size 0.8) (drill 0.4) (layers "F.Cu" "B.Cu") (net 15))
 (via (at 84.836 49.784) (size 0.8) (drill 0.4) (layers "F.Cu" "B.Cu") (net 15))
 (segment (start 87.884 55.88) (end 89.154 54.61) (width 1) (layer "B.Cu") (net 15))
 (segment (start 82.296 52.324) (end 84.836 49.784) (width 1) (layer "B.Cu") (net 15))
 (segment (start 74.93 64.371831) (end 74.93 65.001) (width 1) (layer "B.Cu") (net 15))
 (segment (start 73.66 58.109) (end 73.66 63.101831) (width 1) (layer "B.Cu") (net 15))
 (segment (start 85.344 55.88) (end 87.884 55.88) (width 1) (layer "B.Cu") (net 15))
 (segment (start 73.66 63.101831) (end 74.93 64.371831) (width 1) (layer "B.Cu") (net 15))
 (segment (start 80.01 52.324) (end 82.296 52.324) (width 1) (layer "B.Cu") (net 15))
 (segment (start 64.516 52.072) (end 64.516 48.31) (width 1) (layer "F.Cu") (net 2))
 (segment (start 63.526051 48.31) (end 59.965511 44.74946) (width 1) (layer "B.Cu") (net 2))
 (segment (start 59.965511 40.369381) (end 60.47351 39.861382) (width 1) (layer "B.Cu") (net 2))
 (segment (start 60.47351 39.861382) (end 60.47351 35.08851) (width 1) (layer "B.Cu") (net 2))
 (segment (start 60.47351 35.08851) (end 60.437 35.052) (width 1) (layer "B.Cu") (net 2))
 (segment (start 64.516 48.31) (end 63.526051 48.31) (width 1) (layer "B.Cu") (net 2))
 (segment (start 59.965511 44.74946) (end 59.965511 40.369381) (width 1) (layer "B.Cu") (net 2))
 (segment (start 48.2864 38.5308) (end 51.7652 35.052) (width 1) (layer "F.Cu") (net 18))
 (segment (start 51.7652 35.052) (end 55.357 35.052) (width 1) (layer "F.Cu") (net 18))
 (segment (start 48.2864 40.1811) (end 48.2864 38.5308) (width 1) (layer "F.Cu") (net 18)))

